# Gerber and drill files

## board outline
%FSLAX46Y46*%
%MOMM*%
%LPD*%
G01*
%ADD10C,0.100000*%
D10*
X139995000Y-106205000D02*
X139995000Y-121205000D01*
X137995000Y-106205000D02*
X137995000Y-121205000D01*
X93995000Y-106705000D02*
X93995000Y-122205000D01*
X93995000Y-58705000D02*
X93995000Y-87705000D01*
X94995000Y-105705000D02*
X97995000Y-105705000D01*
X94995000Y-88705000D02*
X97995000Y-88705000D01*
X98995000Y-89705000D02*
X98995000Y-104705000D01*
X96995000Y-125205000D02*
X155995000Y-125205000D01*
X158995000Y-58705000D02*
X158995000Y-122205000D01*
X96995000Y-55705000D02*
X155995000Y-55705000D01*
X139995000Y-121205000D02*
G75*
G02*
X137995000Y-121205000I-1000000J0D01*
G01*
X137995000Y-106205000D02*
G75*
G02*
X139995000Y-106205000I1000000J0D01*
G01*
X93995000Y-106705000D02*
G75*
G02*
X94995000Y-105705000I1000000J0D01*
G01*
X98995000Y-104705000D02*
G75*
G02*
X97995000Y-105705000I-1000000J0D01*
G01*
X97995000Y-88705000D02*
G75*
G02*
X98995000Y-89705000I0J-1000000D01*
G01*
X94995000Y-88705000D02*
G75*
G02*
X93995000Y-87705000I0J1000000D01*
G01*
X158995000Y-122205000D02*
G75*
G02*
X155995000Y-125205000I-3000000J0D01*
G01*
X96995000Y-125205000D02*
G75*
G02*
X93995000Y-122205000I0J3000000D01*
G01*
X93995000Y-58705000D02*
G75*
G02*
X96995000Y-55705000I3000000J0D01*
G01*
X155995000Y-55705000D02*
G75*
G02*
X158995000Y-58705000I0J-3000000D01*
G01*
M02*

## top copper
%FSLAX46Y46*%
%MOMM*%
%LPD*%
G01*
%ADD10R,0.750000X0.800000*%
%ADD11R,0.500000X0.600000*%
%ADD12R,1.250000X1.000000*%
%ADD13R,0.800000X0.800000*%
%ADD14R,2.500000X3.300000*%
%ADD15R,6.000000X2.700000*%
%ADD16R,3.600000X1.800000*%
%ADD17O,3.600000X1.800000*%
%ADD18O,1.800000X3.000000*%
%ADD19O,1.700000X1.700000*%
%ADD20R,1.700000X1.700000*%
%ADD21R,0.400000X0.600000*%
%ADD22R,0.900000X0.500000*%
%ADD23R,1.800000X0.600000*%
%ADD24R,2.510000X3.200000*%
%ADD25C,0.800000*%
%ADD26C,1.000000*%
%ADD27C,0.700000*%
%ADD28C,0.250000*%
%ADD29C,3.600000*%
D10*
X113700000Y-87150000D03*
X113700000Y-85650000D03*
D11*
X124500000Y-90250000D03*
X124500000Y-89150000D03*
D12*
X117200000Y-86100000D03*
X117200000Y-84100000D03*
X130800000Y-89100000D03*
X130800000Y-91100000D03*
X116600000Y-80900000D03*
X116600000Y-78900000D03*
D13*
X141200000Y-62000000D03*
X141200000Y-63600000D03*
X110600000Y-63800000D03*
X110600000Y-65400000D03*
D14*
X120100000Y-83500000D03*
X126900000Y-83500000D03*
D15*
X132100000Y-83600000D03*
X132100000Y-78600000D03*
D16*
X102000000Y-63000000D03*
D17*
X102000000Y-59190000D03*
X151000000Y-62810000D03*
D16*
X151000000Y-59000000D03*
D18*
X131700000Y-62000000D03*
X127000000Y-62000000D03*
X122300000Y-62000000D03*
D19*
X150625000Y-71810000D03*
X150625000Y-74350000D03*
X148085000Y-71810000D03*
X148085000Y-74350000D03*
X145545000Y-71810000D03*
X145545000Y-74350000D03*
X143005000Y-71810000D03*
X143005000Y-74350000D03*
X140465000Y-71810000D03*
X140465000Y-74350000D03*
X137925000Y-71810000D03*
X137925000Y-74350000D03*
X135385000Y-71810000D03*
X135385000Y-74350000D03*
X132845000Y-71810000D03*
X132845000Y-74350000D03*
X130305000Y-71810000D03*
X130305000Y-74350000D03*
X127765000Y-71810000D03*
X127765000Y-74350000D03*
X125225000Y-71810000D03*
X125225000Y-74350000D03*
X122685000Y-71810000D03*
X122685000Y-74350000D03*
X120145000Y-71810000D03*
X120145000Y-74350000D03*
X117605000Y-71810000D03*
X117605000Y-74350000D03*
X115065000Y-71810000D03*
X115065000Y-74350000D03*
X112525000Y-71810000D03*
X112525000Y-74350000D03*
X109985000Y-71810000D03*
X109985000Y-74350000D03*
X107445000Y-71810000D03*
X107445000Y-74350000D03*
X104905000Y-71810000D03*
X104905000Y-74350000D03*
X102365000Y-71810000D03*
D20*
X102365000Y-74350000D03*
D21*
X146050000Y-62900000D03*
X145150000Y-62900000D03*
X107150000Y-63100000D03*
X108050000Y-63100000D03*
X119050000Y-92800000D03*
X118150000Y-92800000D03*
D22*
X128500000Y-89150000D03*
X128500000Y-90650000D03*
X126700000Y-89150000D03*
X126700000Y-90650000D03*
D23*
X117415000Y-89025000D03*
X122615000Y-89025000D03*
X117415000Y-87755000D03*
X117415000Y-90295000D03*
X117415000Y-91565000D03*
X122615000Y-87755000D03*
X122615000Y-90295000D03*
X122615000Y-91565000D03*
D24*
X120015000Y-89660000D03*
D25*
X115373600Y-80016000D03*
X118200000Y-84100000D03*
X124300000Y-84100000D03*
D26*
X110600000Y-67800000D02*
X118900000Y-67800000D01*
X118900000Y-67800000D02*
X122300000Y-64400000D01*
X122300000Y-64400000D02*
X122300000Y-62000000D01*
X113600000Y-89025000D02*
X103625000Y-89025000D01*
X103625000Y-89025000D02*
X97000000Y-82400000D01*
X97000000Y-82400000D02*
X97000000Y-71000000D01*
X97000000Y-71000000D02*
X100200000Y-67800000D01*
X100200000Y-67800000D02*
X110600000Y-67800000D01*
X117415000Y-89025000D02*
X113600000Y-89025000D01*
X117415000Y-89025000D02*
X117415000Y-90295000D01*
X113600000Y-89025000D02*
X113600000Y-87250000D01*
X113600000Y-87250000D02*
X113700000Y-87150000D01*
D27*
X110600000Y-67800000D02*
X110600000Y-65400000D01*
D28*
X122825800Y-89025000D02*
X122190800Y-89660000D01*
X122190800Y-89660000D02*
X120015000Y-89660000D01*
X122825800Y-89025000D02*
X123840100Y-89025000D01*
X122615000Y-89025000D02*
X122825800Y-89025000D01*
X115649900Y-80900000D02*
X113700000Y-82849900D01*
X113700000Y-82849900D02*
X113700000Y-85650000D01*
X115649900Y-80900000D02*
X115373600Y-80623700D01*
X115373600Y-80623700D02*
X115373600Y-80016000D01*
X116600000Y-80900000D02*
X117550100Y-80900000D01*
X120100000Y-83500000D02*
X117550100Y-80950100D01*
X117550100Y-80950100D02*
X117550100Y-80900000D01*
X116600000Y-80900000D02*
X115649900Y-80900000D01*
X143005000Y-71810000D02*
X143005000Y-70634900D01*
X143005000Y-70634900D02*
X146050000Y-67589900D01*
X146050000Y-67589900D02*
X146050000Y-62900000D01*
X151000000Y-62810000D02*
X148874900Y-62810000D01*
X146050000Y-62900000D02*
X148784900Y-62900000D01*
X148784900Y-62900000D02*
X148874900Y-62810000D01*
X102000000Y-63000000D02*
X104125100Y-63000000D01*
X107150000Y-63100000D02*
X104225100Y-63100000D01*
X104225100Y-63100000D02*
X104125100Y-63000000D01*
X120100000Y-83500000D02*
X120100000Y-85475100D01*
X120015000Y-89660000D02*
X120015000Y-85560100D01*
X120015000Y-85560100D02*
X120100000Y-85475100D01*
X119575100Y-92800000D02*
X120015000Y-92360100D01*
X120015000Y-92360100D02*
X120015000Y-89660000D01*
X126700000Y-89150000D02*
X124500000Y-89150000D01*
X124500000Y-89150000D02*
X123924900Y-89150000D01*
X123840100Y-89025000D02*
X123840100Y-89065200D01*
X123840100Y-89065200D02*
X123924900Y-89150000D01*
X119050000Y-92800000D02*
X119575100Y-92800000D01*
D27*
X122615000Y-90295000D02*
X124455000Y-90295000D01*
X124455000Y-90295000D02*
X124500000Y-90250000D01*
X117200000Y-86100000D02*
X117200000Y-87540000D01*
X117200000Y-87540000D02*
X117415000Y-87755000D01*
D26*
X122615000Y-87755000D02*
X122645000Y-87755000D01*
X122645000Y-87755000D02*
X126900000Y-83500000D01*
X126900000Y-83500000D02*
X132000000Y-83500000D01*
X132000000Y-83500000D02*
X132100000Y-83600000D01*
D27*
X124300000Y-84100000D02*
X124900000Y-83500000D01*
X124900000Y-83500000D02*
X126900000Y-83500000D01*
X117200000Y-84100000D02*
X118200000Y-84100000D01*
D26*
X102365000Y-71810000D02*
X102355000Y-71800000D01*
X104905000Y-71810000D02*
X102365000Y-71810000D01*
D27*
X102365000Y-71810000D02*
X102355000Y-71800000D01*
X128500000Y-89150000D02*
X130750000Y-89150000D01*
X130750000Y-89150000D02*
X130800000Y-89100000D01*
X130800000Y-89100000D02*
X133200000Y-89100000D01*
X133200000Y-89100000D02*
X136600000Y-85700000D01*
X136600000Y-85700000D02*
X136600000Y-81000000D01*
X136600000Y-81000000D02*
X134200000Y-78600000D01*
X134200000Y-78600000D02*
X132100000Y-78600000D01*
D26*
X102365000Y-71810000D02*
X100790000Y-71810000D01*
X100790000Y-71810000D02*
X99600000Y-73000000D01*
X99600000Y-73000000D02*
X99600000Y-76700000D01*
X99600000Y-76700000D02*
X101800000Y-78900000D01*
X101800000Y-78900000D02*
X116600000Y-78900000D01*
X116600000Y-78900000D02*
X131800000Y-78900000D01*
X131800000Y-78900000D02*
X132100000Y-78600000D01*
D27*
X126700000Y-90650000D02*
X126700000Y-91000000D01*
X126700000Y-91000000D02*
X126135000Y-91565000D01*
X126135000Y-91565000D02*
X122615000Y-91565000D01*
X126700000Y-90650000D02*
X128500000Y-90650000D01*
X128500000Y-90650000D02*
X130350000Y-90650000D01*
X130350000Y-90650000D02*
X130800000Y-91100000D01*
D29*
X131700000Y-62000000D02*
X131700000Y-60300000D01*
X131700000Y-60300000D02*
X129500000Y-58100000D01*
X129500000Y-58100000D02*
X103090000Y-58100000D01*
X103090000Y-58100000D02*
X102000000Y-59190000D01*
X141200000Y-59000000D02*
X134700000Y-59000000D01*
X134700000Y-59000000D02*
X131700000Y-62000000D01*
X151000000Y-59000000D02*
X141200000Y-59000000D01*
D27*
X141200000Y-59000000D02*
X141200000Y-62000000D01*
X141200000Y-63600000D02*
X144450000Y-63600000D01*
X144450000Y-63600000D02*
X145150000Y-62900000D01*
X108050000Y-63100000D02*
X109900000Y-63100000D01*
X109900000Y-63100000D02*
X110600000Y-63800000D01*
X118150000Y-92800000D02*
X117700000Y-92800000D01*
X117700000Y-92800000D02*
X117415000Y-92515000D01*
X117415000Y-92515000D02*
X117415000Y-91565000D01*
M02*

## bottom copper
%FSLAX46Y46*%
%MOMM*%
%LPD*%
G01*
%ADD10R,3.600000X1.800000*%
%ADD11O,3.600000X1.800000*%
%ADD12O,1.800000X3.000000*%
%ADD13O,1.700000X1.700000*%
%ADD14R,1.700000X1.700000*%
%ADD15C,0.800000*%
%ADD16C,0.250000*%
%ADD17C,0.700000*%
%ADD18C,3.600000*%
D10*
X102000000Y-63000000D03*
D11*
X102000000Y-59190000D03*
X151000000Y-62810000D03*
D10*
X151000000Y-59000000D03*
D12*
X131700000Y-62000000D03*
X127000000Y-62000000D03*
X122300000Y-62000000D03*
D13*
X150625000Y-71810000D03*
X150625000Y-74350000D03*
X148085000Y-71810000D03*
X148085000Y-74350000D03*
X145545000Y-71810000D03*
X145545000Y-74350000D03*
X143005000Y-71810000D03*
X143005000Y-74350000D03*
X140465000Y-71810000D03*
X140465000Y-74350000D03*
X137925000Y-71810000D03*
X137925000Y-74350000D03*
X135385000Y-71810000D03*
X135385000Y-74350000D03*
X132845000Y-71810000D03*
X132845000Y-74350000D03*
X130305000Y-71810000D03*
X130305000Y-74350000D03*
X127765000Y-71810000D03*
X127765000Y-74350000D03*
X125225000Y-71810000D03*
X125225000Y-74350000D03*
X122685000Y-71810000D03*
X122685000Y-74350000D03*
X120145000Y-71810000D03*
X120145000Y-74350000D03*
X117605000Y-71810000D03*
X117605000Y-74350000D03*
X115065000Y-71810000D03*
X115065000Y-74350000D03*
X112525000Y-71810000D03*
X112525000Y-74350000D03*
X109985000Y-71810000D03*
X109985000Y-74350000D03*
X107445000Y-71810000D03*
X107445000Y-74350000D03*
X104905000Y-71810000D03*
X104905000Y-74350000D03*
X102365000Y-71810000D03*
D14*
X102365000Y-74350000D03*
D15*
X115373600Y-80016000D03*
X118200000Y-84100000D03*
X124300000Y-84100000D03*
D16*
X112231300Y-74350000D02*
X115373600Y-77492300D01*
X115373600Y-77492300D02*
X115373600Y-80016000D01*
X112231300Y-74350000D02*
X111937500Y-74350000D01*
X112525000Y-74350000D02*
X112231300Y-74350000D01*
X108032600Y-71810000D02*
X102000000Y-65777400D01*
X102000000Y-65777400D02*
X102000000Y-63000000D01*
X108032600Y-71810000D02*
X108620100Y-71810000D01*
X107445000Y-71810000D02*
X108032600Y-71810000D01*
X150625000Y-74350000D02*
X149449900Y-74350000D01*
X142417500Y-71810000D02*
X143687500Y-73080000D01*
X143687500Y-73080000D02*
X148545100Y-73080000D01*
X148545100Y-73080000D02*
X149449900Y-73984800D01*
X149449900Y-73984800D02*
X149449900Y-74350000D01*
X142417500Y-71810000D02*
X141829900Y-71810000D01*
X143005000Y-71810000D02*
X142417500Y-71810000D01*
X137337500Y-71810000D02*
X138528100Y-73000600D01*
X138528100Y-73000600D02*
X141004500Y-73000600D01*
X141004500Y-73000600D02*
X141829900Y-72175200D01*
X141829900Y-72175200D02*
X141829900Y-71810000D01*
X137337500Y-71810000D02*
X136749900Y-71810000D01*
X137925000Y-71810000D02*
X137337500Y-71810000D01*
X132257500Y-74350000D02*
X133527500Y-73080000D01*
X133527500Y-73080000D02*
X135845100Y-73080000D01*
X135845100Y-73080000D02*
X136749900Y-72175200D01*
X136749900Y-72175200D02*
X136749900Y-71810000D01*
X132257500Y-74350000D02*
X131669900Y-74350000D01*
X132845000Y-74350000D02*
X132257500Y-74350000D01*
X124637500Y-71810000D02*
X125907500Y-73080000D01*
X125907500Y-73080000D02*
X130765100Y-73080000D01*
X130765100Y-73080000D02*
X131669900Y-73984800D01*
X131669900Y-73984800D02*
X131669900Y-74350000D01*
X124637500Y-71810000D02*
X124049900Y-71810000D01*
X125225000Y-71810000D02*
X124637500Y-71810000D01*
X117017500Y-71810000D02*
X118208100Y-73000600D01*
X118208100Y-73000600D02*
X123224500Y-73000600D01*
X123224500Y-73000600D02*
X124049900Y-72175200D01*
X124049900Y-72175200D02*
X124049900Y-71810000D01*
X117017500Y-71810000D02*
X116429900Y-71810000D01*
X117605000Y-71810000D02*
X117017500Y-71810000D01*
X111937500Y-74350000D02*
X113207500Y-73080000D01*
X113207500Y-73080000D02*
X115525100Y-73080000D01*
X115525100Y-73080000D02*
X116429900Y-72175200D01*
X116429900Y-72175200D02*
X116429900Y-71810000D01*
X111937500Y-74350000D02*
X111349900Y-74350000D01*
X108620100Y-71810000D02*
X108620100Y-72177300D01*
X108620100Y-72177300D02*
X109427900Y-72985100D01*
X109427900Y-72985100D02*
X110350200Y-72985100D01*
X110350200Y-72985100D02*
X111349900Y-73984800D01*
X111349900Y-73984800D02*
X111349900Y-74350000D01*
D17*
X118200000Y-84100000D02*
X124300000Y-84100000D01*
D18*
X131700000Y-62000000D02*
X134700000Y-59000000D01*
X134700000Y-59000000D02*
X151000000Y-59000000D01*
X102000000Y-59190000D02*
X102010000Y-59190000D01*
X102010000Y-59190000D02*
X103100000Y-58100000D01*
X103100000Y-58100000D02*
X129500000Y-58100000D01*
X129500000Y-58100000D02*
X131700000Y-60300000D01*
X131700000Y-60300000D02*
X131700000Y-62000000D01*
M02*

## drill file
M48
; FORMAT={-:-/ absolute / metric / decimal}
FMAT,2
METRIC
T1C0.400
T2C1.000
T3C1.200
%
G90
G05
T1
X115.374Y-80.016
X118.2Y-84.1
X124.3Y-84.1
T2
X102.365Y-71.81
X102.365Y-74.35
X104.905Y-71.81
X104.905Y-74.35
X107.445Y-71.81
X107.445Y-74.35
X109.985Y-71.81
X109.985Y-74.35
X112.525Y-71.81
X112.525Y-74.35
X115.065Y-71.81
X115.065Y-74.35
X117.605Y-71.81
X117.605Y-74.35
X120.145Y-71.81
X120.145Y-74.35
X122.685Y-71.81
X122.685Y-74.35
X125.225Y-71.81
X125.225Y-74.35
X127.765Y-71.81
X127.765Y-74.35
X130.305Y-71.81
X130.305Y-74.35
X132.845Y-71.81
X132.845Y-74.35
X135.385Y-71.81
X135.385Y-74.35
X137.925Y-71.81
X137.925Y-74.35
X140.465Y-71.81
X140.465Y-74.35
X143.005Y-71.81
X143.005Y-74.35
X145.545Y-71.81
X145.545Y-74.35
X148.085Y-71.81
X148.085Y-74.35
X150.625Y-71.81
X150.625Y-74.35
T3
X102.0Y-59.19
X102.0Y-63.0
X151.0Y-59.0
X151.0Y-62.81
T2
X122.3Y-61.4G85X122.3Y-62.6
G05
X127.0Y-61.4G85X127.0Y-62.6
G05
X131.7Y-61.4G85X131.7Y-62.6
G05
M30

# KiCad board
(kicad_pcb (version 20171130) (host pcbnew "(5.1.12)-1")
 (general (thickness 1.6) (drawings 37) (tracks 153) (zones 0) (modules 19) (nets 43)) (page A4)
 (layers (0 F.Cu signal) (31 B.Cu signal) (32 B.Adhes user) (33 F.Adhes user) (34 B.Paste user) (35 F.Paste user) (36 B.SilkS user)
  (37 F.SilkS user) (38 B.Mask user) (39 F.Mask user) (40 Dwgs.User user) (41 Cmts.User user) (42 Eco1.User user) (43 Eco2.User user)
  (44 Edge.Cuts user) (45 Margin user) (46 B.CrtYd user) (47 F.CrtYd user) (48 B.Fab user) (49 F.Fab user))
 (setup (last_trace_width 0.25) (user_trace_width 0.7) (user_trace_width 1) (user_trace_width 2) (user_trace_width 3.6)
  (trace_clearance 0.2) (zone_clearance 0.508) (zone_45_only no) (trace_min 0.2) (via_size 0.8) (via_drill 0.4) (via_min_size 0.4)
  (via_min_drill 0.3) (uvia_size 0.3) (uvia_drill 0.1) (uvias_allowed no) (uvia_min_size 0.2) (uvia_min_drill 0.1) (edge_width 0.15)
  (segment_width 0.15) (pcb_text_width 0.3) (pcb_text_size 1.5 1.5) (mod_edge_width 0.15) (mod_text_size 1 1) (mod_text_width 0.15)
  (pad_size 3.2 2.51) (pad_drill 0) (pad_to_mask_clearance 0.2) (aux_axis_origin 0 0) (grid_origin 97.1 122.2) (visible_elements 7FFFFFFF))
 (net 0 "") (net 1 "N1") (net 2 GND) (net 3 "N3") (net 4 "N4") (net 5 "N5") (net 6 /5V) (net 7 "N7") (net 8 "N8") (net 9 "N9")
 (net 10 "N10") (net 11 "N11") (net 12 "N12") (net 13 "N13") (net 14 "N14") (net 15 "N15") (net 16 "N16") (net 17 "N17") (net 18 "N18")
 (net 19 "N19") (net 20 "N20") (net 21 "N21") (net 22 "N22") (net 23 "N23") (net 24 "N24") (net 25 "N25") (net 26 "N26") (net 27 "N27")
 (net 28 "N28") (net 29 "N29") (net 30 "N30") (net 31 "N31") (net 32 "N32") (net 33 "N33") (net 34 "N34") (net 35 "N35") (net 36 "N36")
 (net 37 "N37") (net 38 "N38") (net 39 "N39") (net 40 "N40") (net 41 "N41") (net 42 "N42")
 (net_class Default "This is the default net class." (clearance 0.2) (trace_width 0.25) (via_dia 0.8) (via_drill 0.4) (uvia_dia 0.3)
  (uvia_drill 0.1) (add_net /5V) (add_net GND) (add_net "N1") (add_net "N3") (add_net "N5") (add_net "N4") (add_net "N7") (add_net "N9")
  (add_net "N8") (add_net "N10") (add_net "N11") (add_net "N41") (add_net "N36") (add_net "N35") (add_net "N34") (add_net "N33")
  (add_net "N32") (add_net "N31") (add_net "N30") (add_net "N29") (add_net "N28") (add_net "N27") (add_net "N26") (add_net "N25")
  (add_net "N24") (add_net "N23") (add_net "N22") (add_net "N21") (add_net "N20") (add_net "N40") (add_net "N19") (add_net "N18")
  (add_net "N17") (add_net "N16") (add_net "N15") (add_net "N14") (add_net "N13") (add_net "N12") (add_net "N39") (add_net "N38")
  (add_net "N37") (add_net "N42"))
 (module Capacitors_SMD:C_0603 (layer F.Cu) (at 113.7 86.4 270)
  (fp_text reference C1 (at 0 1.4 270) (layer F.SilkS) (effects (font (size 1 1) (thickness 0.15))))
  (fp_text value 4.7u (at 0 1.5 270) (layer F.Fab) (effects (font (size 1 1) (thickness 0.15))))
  (pad 2 smd rect (at 0.75 0 270) (size 0.8 0.75) (layers F.Cu F.Paste F.Mask) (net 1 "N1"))
  (pad 1 smd rect (at -0.75 0 270) (size 0.8 0.75) (layers F.Cu F.Paste F.Mask) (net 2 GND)))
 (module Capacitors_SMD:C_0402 (layer F.Cu) (at 124.5 89.7 270)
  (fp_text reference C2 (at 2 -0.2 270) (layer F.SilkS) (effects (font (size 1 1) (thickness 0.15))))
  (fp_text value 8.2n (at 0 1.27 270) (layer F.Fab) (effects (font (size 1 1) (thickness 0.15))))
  (pad 2 smd rect (at 0.55 0 270) (size 0.6 0.5) (layers F.Cu F.Paste F.Mask) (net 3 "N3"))
  (pad 1 smd rect (at -0.55 0 270) (size 0.6 0.5) (layers F.Cu F.Paste F.Mask) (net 2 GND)))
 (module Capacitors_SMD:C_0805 (layer F.Cu) (at 117.2 85.1 270)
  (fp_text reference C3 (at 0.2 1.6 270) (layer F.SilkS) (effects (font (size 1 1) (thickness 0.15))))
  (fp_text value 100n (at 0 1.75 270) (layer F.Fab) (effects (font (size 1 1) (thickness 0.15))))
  (pad 2 smd rect (at 1 0 270) (size 1 1.25) (layers F.Cu F.Paste F.Mask) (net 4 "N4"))
  (pad 1 smd rect (at -1 0 270) (size 1 1.25) (layers F.Cu F.Paste F.Mask) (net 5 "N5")))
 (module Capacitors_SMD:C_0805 (layer F.Cu) (at 130.8 90.1 90)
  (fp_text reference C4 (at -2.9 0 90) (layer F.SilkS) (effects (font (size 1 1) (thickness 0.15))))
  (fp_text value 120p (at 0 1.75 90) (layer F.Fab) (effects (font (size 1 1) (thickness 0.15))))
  (pad 2 smd rect (at 1 0 90) (size 1 1.25) (layers F.Cu F.Paste F.Mask) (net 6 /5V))
  (pad 1 smd rect (at -1 0 90) (size 1 1.25) (layers F.Cu F.Paste F.Mask) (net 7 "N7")))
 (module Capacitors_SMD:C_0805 (layer F.Cu) (at 116.6 79.9 90)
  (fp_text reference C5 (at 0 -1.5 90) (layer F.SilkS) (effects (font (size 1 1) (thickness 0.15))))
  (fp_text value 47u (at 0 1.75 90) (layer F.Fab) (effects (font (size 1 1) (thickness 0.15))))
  (pad 1 smd rect (at -1 0 90) (size 1 1.25) (layers F.Cu F.Paste F.Mask) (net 2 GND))
  (pad 2 smd rect (at 1 0 90) (size 1 1.25) (layers F.Cu F.Paste F.Mask) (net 6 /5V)))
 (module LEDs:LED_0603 (layer F.Cu) (at 141.2 62.8 90)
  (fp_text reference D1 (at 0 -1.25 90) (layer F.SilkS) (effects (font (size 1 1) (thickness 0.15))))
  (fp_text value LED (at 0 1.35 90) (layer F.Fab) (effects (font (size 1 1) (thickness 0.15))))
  (pad 2 smd rect (at 0.8 0 270) (size 0.8 0.8) (layers F.Cu F.Paste F.Mask) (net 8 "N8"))
  (pad 1 smd rect (at -0.8 0 270) (size 0.8 0.8) (layers F.Cu F.Paste F.Mask) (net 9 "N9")))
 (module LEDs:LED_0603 (layer F.Cu) (at 110.6 64.6 270)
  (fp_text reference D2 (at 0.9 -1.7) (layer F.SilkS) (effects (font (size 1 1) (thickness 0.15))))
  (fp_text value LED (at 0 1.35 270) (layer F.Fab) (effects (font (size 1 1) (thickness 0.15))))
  (pad 1 smd rect (at -0.8 0 90) (size 0.8 0.8) (layers F.Cu F.Paste F.Mask) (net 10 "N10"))
  (pad 2 smd rect (at 0.8 0 90) (size 0.8 0.8) (layers F.Cu F.Paste F.Mask) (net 1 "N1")))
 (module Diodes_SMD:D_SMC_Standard (layer F.Cu) (at 123.5 83.5 180)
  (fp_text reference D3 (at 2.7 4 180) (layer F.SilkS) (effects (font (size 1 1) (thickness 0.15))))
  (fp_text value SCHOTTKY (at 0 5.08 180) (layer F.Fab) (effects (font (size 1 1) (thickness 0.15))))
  (pad 2 smd rect (at 3.4 0 270) (size 3.3 2.5) (layers F.Cu F.Paste F.Mask) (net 2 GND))
  (pad 1 smd rect (at -3.4 0 270) (size 3.3 2.5) (layers F.Cu F.Paste F.Mask) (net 5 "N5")))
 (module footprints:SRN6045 (layer F.Cu) (at 132.1 81.1 270)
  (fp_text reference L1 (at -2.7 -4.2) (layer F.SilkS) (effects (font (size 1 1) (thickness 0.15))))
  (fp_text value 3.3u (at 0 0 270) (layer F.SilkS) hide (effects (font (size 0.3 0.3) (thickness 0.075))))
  (pad 2 smd rect (at 2.5 0 270) (size 2.7 6) (layers F.Cu F.Paste F.Mask) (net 5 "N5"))
  (pad 1 smd rect (at -2.5 0 270) (size 2.7 6) (layers F.Cu F.Paste F.Mask) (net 6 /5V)))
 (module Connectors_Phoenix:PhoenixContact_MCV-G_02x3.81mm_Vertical (layer F.Cu) (at 102 63 90)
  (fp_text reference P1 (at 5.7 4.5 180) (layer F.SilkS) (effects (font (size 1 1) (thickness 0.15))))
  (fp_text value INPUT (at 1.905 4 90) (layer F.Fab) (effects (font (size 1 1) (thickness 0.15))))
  (pad 1 thru_hole rect (at 0 0 90) (size 1.8 3.6) (drill 1.2) (layers *.Cu *.Mask) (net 2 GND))
  (pad 2 thru_hole oval (at 3.81 0 90) (size 1.8 3.6) (drill 1.2) (layers *.Cu *.Mask) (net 8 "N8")))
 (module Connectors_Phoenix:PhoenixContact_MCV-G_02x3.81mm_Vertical (layer F.Cu) (at 151 59 270)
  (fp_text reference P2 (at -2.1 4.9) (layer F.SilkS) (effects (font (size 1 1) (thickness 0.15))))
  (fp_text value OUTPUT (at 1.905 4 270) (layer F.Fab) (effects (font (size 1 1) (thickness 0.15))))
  (pad 2 thru_hole oval (at 3.81 0 270) (size 1.8 3.6) (drill 1.2) (layers *.Cu *.Mask) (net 2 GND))
  (pad 1 thru_hole rect (at 0 0 270) (size 1.8 3.6) (drill 1.2) (layers *.Cu *.Mask) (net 8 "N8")))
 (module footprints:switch (layer F.Cu) (at 127 62)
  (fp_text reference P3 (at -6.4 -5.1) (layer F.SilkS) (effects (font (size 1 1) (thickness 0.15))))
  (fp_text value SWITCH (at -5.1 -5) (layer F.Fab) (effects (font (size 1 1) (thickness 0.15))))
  (pad 3 thru_hole oval (at 4.7 0) (size 1.8 3) (drill oval 1 2.2) (layers *.Cu *.Mask) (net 8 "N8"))
  (pad 2 thru_hole oval (at 0 0) (size 1.8 3) (drill oval 1 2.2) (layers *.Cu *.Mask) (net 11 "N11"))
  (pad 1 thru_hole oval (at -4.7 0) (size 1.8 3) (drill oval 1 2.2) (layers *.Cu *.Mask) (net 1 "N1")))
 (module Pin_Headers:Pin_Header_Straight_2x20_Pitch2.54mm (layer F.Cu) (at 102.365 74.35 90)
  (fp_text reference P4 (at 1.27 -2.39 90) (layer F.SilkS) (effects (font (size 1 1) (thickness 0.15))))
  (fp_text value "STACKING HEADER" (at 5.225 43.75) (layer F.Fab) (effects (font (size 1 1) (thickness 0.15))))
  (pad 40 thru_hole oval (at 2.54 48.26 90) (size 1.7 1.7) (drill 1) (layers *.Cu *.Mask) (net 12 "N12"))
  (pad 39 thru_hole oval (at 0 48.26 90) (size 1.7 1.7) (drill 1) (layers *.Cu *.Mask) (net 2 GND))
  (pad 38 thru_hole oval (at 2.54 45.72 90) (size 1.7 1.7) (drill 1) (layers *.Cu *.Mask) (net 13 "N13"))
  (pad 37 thru_hole oval (at 0 45.72 90) (size 1.7 1.7) (drill 1) (layers *.Cu *.Mask) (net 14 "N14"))
  (pad 36 thru_hole oval (at 2.54 43.18 90) (size 1.7 1.7) (drill 1) (layers *.Cu *.Mask) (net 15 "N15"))
  (pad 35 thru_hole oval (at 0 43.18 90) (size 1.7 1.7) (drill 1) (layers *.Cu *.Mask) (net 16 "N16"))
  (pad 34 thru_hole oval (at 2.54 40.64 90) (size 1.7 1.7) (drill 1) (layers *.Cu *.Mask) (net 2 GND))
  (pad 33 thru_hole oval (at 0 40.64 90) (size 1.7 1.7) (drill 1) (layers *.Cu *.Mask) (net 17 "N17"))
  (pad 32 thru_hole oval (at 2.54 38.1 90) (size 1.7 1.7) (drill 1) (layers *.Cu *.Mask) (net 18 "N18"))
  (pad 31 thru_hole oval (at 0 38.1 90) (size 1.7 1.7) (drill 1) (layers *.Cu *.Mask) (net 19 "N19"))
  (pad 30 thru_hole oval (at 2.54 35.56 90) (size 1.7 1.7) (drill 1) (layers *.Cu *.Mask) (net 2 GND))
  (pad 29 thru_hole oval (at 0 35.56 90) (size 1.7 1.7) (drill 1) (layers *.Cu *.Mask) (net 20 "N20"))
  (pad 28 thru_hole oval (at 2.54 33.02 90) (size 1.7 1.7) (drill 1) (layers *.Cu *.Mask) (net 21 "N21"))
  (pad 27 thru_hole oval (at 0 33.02 90) (size 1.7 1.7) (drill 1) (layers *.Cu *.Mask) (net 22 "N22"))
  (pad 26 thru_hole oval (at 2.54 30.48 90) (size 1.7 1.7) (drill 1) (layers *.Cu *.Mask) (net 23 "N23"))
  (pad 25 thru_hole oval (at 0 30.48 90) (size 1.7 1.7) (drill 1) (layers *.Cu *.Mask) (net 2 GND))
  (pad 24 thru_hole oval (at 2.54 27.94 90) (size 1.7 1.7) (drill 1) (layers *.Cu *.Mask) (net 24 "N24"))
  (pad 23 thru_hole oval (at 0 27.94 90) (size 1.7 1.7) (drill 1) (layers *.Cu *.Mask) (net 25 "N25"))
  (pad 22 thru_hole oval (at 2.54 25.4 90) (size 1.7 1.7) (drill 1) (layers *.Cu *.Mask) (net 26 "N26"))
  (pad 21 thru_hole oval (at 0 25.4 90) (size 1.7 1.7) (drill 1) (layers *.Cu *.Mask) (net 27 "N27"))
  (pad 20 thru_hole oval (at 2.54 22.86 90) (size 1.7 1.7) (drill 1) (layers *.Cu *.Mask) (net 2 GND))
  (pad 19 thru_hole oval (at 0 22.86 90) (size 1.7 1.7) (drill 1) (layers *.Cu *.Mask) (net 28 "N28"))
  (pad 18 thru_hole oval (at 2.54 20.32 90) (size 1.7 1.7) (drill 1) (layers *.Cu *.Mask) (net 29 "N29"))
  (pad 17 thru_hole oval (at 0 20.32 90) (size 1.7 1.7) (drill 1) (layers *.Cu *.Mask) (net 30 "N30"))
  (pad 16 thru_hole oval (at 2.54 17.78 90) (size 1.7 1.7) (drill 1) (layers *.Cu *.Mask) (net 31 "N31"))
  (pad 15 thru_hole oval (at 0 17.78 90) (size 1.7 1.7) (drill 1) (layers *.Cu *.Mask) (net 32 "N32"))
  (pad 14 thru_hole oval (at 2.54 15.24 90) (size 1.7 1.7) (drill 1) (layers *.Cu *.Mask) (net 2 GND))
  (pad 13 thru_hole oval (at 0 15.24 90) (size 1.7 1.7) (drill 1) (layers *.Cu *.Mask) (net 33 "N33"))
  (pad 12 thru_hole oval (at 2.54 12.7 90) (size 1.7 1.7) (drill 1) (layers *.Cu *.Mask) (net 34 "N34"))
  (pad 11 thru_hole oval (at 0 12.7 90) (size 1.7 1.7) (drill 1) (layers *.Cu *.Mask) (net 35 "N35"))
  (pad 10 thru_hole oval (at 2.54 10.16 90) (size 1.7 1.7) (drill 1) (layers *.Cu *.Mask) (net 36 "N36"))
  (pad 9 thru_hole oval (at 0 10.16 90) (size 1.7 1.7) (drill 1) (layers *.Cu *.Mask) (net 2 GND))
  (pad 8 thru_hole oval (at 2.54 7.62 90) (size 1.7 1.7) (drill 1) (layers *.Cu *.Mask) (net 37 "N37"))
  (pad 7 thru_hole oval (at 0 7.62 90) (size 1.7 1.7) (drill 1) (layers *.Cu *.Mask) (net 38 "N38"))
  (pad 6 thru_hole oval (at 2.54 5.08 90) (size 1.7 1.7) (drill 1) (layers *.Cu *.Mask) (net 2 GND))
  (pad 5 thru_hole oval (at 0 5.08 90) (size 1.7 1.7) (drill 1) (layers *.Cu *.Mask) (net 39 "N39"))
  (pad 4 thru_hole oval (at 2.54 2.54 90) (size 1.7 1.7) (drill 1) (layers *.Cu *.Mask) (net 6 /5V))
  (pad 3 thru_hole oval (at 0 2.54 90) (size 1.7 1.7) (drill 1) (layers *.Cu *.Mask) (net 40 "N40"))
  (pad 2 thru_hole oval (at 2.54 0 90) (size 1.7 1.7) (drill 1) (layers *.Cu *.Mask) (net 6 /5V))
  (pad 1 thru_hole rect (at 0 0 90) (size 1.7 1.7) (drill 1) (layers *.Cu *.Mask) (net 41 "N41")))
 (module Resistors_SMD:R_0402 (layer F.Cu) (at 145.6 62.9)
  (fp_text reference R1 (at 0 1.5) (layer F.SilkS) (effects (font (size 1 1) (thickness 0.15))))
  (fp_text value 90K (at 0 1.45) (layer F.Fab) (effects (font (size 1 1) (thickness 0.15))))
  (pad 2 smd rect (at 0.45 0) (size 0.4 0.6) (layers F.Cu F.Paste F.Mask) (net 2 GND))
  (pad 1 smd rect (at -0.45 0) (size 0.4 0.6) (layers F.Cu F.Paste F.Mask) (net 9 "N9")))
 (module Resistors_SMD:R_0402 (layer F.Cu) (at 107.6 63.1 180)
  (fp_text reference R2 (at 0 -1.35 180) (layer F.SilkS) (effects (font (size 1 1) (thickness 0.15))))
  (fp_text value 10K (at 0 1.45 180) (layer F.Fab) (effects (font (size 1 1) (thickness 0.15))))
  (pad 2 smd rect (at 0.45 0 180) (size 0.4 0.6) (layers F.Cu F.Paste F.Mask) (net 2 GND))
  (pad 1 smd rect (at -0.45 0 180) (size 0.4 0.6) (layers F.Cu F.Paste F.Mask) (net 10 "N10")))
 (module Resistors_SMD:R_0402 (layer F.Cu) (at 118.6 92.8)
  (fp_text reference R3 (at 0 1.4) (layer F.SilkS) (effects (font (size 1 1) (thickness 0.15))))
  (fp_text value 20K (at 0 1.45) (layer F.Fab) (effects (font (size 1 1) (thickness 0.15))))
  (pad 2 smd rect (at 0.45 0) (size 0.4 0.6) (layers F.Cu F.Paste F.Mask) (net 2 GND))
  (pad 1 smd rect (at -0.45 0) (size 0.4 0.6) (layers F.Cu F.Paste F.Mask) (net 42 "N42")))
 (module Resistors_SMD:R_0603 (layer F.Cu) (at 128.5 89.9 270)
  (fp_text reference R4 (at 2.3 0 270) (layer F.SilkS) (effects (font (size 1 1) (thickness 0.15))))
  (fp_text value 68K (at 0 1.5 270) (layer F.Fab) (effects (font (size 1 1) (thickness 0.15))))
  (pad 1 smd rect (at -0.75 0 270) (size 0.5 0.9) (layers F.Cu F.Paste F.Mask) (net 6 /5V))
  (pad 2 smd rect (at 0.75 0 270) (size 0.5 0.9) (layers F.Cu F.Paste F.Mask) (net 7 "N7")))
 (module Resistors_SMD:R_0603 (layer F.Cu) (at 126.7 89.9 90)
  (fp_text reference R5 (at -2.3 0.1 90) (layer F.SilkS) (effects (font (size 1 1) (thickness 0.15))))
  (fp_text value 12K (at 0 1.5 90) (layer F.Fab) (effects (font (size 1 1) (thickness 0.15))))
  (pad 2 smd rect (at 0.75 0 90) (size 0.5 0.9) (layers F.Cu F.Paste F.Mask) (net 2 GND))
  (pad 1 smd rect (at -0.75 0 90) (size 0.5 0.9) (layers F.Cu F.Paste F.Mask) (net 7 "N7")))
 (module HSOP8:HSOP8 (layer F.Cu) (at 120.015 89.66 270) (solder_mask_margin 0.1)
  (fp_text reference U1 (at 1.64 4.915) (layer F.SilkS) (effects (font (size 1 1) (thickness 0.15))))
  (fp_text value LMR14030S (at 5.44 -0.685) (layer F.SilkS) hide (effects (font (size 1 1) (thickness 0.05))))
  (pad 2 smd rect (at -0.635 2.6 270) (size 0.6 1.8) (layers F.Cu F.Paste F.Mask) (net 1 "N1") (solder_mask_margin 0.2))
  (pad 7 smd rect (at -0.635 -2.6 270) (size 0.6 1.8) (layers F.Cu F.Paste F.Mask) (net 2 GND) (solder_mask_margin 0.2))
  (pad 1 smd rect (at -1.905 2.6 270) (size 0.6 1.8) (layers F.Cu F.Paste F.Mask) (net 4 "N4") (solder_mask_margin 0.2))
  (pad 3 smd rect (at 0.635 2.6 270) (size 0.6 1.8) (layers F.Cu F.Paste F.Mask) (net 1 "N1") (solder_mask_margin 0.2))
  (pad 4 smd rect (at 1.905 2.6 270) (size 0.6 1.8) (layers F.Cu F.Paste F.Mask) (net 42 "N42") (solder_mask_margin 0.2))
  (pad 8 smd rect (at -1.905 -2.6 270) (size 0.6 1.8) (layers F.Cu F.Paste F.Mask) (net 5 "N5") (solder_mask_margin 0.2))
  (pad 6 smd rect (at 0.635 -2.6 270) (size 0.6 1.8) (layers F.Cu F.Paste F.Mask) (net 3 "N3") (solder_mask_margin 0.2))
  (pad 5 smd rect (at 1.905 -2.6 270) (size 0.6 1.8) (layers F.Cu F.Paste F.Mask) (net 7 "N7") (solder_mask_margin 0.2))
  (pad 9 smd rect (at 0 0 270) (size 3.2 2.51) (layers F.Cu F.Paste F.Mask) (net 2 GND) (solder_mask_margin 0.2)))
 (gr_line (start 139.995 106.205) (end 139.995 121.205) (angle 90) (layer Edge.Cuts) (width 0.1))
 (gr_line (start 137.995 106.205) (end 137.995 121.205) (angle 90) (layer Edge.Cuts) (width 0.1))
 (gr_line (start 93.995 106.705) (end 93.995 122.205) (layer Edge.Cuts) (width 0.1))
 (gr_line (start 93.995 58.705) (end 93.995 87.705) (layer Edge.Cuts) (width 0.1))
 (gr_line (start 94.995 105.705) (end 97.995 105.705) (layer Edge.Cuts) (width 0.1))
 (gr_line (start 94.995 88.705) (end 97.995 88.705) (layer Edge.Cuts) (width 0.1))
 (gr_line (start 98.995 89.705) (end 98.995 104.705) (layer Edge.Cuts) (width 0.1))
 (gr_line (start 96.995 125.205) (end 155.995 125.205) (angle 90) (layer Edge.Cuts) (width 0.1))
 (gr_line (start 158.995 58.705) (end 158.995 122.205) (angle 90) (layer Edge.Cuts) (width 0.1))
 (gr_line (start 96.995 55.705) (end 155.995 55.705) (angle 90) (layer Edge.Cuts) (width 0.1))
 (gr_arc (start 138.995 121.205) (end 137.995 121.205) (angle -180) (layer Edge.Cuts) (width 0.1))
 (gr_arc (start 138.995 106.205) (end 137.995 106.205) (angle 180) (layer Edge.Cuts) (width 0.1))
 (gr_arc (start 94.995 106.705) (end 93.995 106.705) (angle 90) (layer Edge.Cuts) (width 0.1))
 (gr_arc (start 97.995 104.705) (end 98.995 104.705) (angle 90) (layer Edge.Cuts) (width 0.1))
 (gr_arc (start 97.995 89.705) (end 97.995 88.705) (angle 90) (layer Edge.Cuts) (width 0.1))
 (gr_arc (start 94.995 87.705) (end 94.995 88.705) (angle 90) (layer Edge.Cuts) (width 0.1))
 (gr_arc (start 155.995 122.205) (end 158.995 122.205) (angle 90) (layer Edge.Cuts) (width 0.1))
 (gr_arc (start 96.995 122.205) (end 96.995 125.205) (angle 90) (layer Edge.Cuts) (width 0.1))
 (gr_arc (start 96.995 58.705) (end 93.995 58.705) (angle 90) (layer Edge.Cuts) (width 0.1))
 (gr_arc (start 155.995 58.705) (end 155.995 55.705) (angle 90) (layer Edge.Cuts) (width 0.1))
 (segment (start 110.6 67.8) (end 118.9 67.8) (width 1) (layer F.Cu) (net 1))
 (segment (start 118.9 67.8) (end 122.3 64.4) (width 1) (layer F.Cu) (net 1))
 (segment (start 122.3 64.4) (end 122.3 62) (width 1) (layer F.Cu) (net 1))
 (segment (start 113.6 89.025) (end 103.625 89.025) (width 1) (layer F.Cu) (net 1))
 (segment (start 103.625 89.025) (end 97 82.4) (width 1) (layer F.Cu) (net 1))
 (segment (start 97 82.4) (end 97 71) (width 1) (layer F.Cu) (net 1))
 (segment (start 97 71) (end 100.2 67.8) (width 1) (layer F.Cu) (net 1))
 (segment (start 100.2 67.8) (end 110.6 67.8) (width 1) (layer F.Cu) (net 1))
 (segment (start 117.415 89.025) (end 113.6 89.025) (width 1) (layer F.Cu) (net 1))
 (segment (start 117.415 89.025) (end 117.415 90.295) (width 1) (layer F.Cu) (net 1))
 (segment (start 113.6 89.025) (end 113.6 87.25) (width 1) (layer F.Cu) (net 1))
 (segment (start 113.6 87.25) (end 113.7 87.15) (width 1) (layer F.Cu) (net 1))
 (segment (start 110.6 67.8) (end 110.6 65.4) (width 0.7) (layer F.Cu) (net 1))
 (segment (start 122.8258 89.025) (end 122.1908 89.66) (width 0.25) (layer F.Cu) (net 2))
 (segment (start 122.1908 89.66) (end 120.015 89.66) (width 0.25) (layer F.Cu) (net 2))
 (segment (start 122.8258 89.025) (end 123.8401 89.025) (width 0.25) (layer F.Cu) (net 2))
 (segment (start 122.615 89.025) (end 122.8258 89.025) (width 0.25) (layer F.Cu) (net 2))
 (segment (start 115.6499 80.9) (end 113.7 82.8499) (width 0.25) (layer F.Cu) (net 2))
 (segment (start 113.7 82.8499) (end 113.7 85.65) (width 0.25) (layer F.Cu) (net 2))
 (segment (start 115.6499 80.9) (end 115.3736 80.6237) (width 0.25) (layer F.Cu) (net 2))
 (segment (start 115.3736 80.6237) (end 115.3736 80.016) (width 0.25) (layer F.Cu) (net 2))
 (segment (start 116.6 80.9) (end 117.5501 80.9) (width 0.25) (layer F.Cu) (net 2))
 (segment (start 120.1 83.5) (end 117.5501 80.9501) (width 0.25) (layer F.Cu) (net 2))
 (segment (start 117.5501 80.9501) (end 117.5501 80.9) (width 0.25) (layer F.Cu) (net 2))
 (segment (start 112.2313 74.35) (end 115.3736 77.4923) (width 0.25) (layer B.Cu) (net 2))
 (segment (start 115.3736 77.4923) (end 115.3736 80.016) (width 0.25) (layer B.Cu) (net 2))
 (segment (start 116.6 80.9) (end 115.6499 80.9) (width 0.25) (layer F.Cu) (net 2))
 (segment (start 112.2313 74.35) (end 111.9375 74.35) (width 0.25) (layer B.Cu) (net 2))
 (segment (start 112.525 74.35) (end 112.2313 74.35) (width 0.25) (layer B.Cu) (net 2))
 (segment (start 108.0326 71.81) (end 102 65.7774) (width 0.25) (layer B.Cu) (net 2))
 (segment (start 102 65.7774) (end 102 63) (width 0.25) (layer B.Cu) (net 2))
 (segment (start 108.0326 71.81) (end 108.6201 71.81) (width 0.25) (layer B.Cu) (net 2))
 (segment (start 107.445 71.81) (end 108.0326 71.81) (width 0.25) (layer B.Cu) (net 2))
 (segment (start 143.005 71.81) (end 143.005 70.6349) (width 0.25) (layer F.Cu) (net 2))
 (segment (start 143.005 70.6349) (end 146.05 67.5899) (width 0.25) (layer F.Cu) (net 2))
 (segment (start 146.05 67.5899) (end 146.05 62.9) (width 0.25) (layer F.Cu) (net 2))
 (segment (start 150.625 74.35) (end 149.4499 74.35) (width 0.25) (layer B.Cu) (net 2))
 (segment (start 142.4175 71.81) (end 143.6875 73.08) (width 0.25) (layer B.Cu) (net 2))
 (segment (start 143.6875 73.08) (end 148.5451 73.08) (width 0.25) (layer B.Cu) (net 2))
 (segment (start 148.5451 73.08) (end 149.4499 73.9848) (width 0.25) (layer B.Cu) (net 2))
 (segment (start 149.4499 73.9848) (end 149.4499 74.35) (width 0.25) (layer B.Cu) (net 2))
 (segment (start 142.4175 71.81) (end 141.8299 71.81) (width 0.25) (layer B.Cu) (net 2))
 (segment (start 143.005 71.81) (end 142.4175 71.81) (width 0.25) (layer B.Cu) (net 2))
 (segment (start 137.3375 71.81) (end 138.5281 73.0006) (width 0.25) (layer B.Cu) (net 2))
 (segment (start 138.5281 73.0006) (end 141.0045 73.0006) (width 0.25) (layer B.Cu) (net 2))
 (segment (start 141.0045 73.0006) (end 141.8299 72.1752) (width 0.25) (layer B.Cu) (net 2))
 (segment (start 141.8299 72.1752) (end 141.8299 71.81) (width 0.25) (layer B.Cu) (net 2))
 (segment (start 137.3375 71.81) (end 136.7499 71.81) (width 0.25) (layer B.Cu) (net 2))
 (segment (start 137.925 71.81) (end 137.3375 71.81) (width 0.25) (layer B.Cu) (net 2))
 (segment (start 132.2575 74.35) (end 133.5275 73.08) (width 0.25) (layer B.Cu) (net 2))
 (segment (start 133.5275 73.08) (end 135.8451 73.08) (width 0.25) (layer B.Cu) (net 2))
 (segment (start 135.8451 73.08) (end 136.7499 72.1752) (width 0.25) (layer B.Cu) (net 2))
 (segment (start 136.7499 72.1752) (end 136.7499 71.81) (width 0.25) (layer B.Cu) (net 2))
 (segment (start 132.2575 74.35) (end 131.6699 74.35) (width 0.25) (layer B.Cu) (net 2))
 (segment (start 132.845 74.35) (end 132.2575 74.35) (width 0.25) (layer B.Cu) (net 2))
 (segment (start 124.6375 71.81) (end 125.9075 73.08) (width 0.25) (layer B.Cu) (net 2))
 (segment (start 125.9075 73.08) (end 130.7651 73.08) (width 0.25) (layer B.Cu) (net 2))
 (segment (start 130.7651 73.08) (end 131.6699 73.9848) (width 0.25) (layer B.Cu) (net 2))
 (segment (start 131.6699 73.9848) (end 131.6699 74.35) (width 0.25) (layer B.Cu) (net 2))
 (segment (start 124.6375 71.81) (end 124.0499 71.81) (width 0.25) (layer B.Cu) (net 2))
 (segment (start 125.225 71.81) (end 124.6375 71.81) (width 0.25) (layer B.Cu) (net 2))
 (segment (start 117.0175 71.81) (end 118.2081 73.0006) (width 0.25) (layer B.Cu) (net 2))
 (segment (start 118.2081 73.0006) (end 123.2245 73.0006) (width 0.25) (layer B.Cu) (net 2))
 (segment (start 123.2245 73.0006) (end 124.0499 72.1752) (width 0.25) (layer B.Cu) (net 2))
 (segment (start 124.0499 72.1752) (end 124.0499 71.81) (width 0.25) (layer B.Cu) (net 2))
 (segment (start 117.0175 71.81) (end 116.4299 71.81) (width 0.25) (layer B.Cu) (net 2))
 (segment (start 117.605 71.81) (end 117.0175 71.81) (width 0.25) (layer B.Cu) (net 2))
 (segment (start 111.9375 74.35) (end 113.2075 73.08) (width 0.25) (layer B.Cu) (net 2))
 (segment (start 113.2075 73.08) (end 115.5251 73.08) (width 0.25) (layer B.Cu) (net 2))
 (segment (start 115.5251 73.08) (end 116.4299 72.1752) (width 0.25) (layer B.Cu) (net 2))
 (segment (start 116.4299 72.1752) (end 116.4299 71.81) (width 0.25) (layer B.Cu) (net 2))
 (segment (start 111.9375 74.35) (end 111.3499 74.35) (width 0.25) (layer B.Cu) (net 2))
 (segment (start 108.6201 71.81) (end 108.6201 72.1773) (width 0.25) (layer B.Cu) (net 2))
 (segment (start 108.6201 72.1773) (end 109.4279 72.9851) (width 0.25) (layer B.Cu) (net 2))
 (segment (start 109.4279 72.9851) (end 110.3502 72.9851) (width 0.25) (layer B.Cu) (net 2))
 (segment (start 110.3502 72.9851) (end 111.3499 73.9848) (width 0.25) (layer B.Cu) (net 2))
 (segment (start 111.3499 73.9848) (end 111.3499 74.35) (width 0.25) (layer B.Cu) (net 2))
 (segment (start 151 62.81) (end 148.8749 62.81) (width 0.25) (layer F.Cu) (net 2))
 (segment (start 146.05 62.9) (end 148.7849 62.9) (width 0.25) (layer F.Cu) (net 2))
 (segment (start 148.7849 62.9) (end 148.8749 62.81) (width 0.25) (layer F.Cu) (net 2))
 (segment (start 102 63) (end 104.1251 63) (width 0.25) (layer F.Cu) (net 2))
 (segment (start 107.15 63.1) (end 104.2251 63.1) (width 0.25) (layer F.Cu) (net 2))
 (segment (start 104.2251 63.1) (end 104.1251 63) (width 0.25) (layer F.Cu) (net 2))
 (segment (start 120.1 83.5) (end 120.1 85.4751) (width 0.25) (layer F.Cu) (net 2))
 (segment (start 120.015 89.66) (end 120.015 85.5601) (width 0.25) (layer F.Cu) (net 2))
 (segment (start 120.015 85.5601) (end 120.1 85.4751) (width 0.25) (layer F.Cu) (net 2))
 (segment (start 119.5751 92.8) (end 120.015 92.3601) (width 0.25) (layer F.Cu) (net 2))
 (segment (start 120.015 92.3601) (end 120.015 89.66) (width 0.25) (layer F.Cu) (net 2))
 (segment (start 126.7 89.15) (end 124.5 89.15) (width 0.25) (layer F.Cu) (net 2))
 (segment (start 124.5 89.15) (end 123.9249 89.15) (width 0.25) (layer F.Cu) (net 2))
 (segment (start 123.8401 89.025) (end 123.8401 89.0652) (width 0.25) (layer F.Cu) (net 2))
 (segment (start 123.8401 89.0652) (end 123.9249 89.15) (width 0.25) (layer F.Cu) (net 2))
 (segment (start 119.05 92.8) (end 119.5751 92.8) (width 0.25) (layer F.Cu) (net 2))
 (via (at 115.3736 80.016) (size 0.8) (layers F.Cu B.Cu) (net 2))
 (segment (start 122.615 90.295) (end 124.455 90.295) (width 0.7) (layer F.Cu) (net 3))
 (segment (start 124.455 90.295) (end 124.5 90.25) (width 0.7) (layer F.Cu) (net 3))
 (segment (start 117.2 86.1) (end 117.2 87.54) (width 0.7) (layer F.Cu) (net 4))
 (segment (start 117.2 87.54) (end 117.415 87.755) (width 0.7) (layer F.Cu) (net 4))
 (segment (start 122.615 87.755) (end 122.645 87.755) (width 1) (layer F.Cu) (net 5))
 (segment (start 122.645 87.755) (end 126.9 83.5) (width 1) (layer F.Cu) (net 5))
 (segment (start 126.9 83.5) (end 132 83.5) (width 1) (layer F.Cu) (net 5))
 (segment (start 132 83.5) (end 132.1 83.6) (width 1) (layer F.Cu) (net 5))
 (segment (start 118.2 84.1) (end 124.3 84.1) (width 0.7) (layer B.Cu) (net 5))
 (segment (start 124.3 84.1) (end 124.9 83.5) (width 0.7) (layer F.Cu) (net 5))
 (segment (start 124.9 83.5) (end 126.9 83.5) (width 0.7) (layer F.Cu) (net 5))
 (segment (start 117.2 84.1) (end 118.2 84.1) (width 0.7) (layer F.Cu) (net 5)) (via (at 118.2 84.1) (size 0.8) (layers F.Cu B.Cu) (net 5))
 (via (at 124.3 84.1) (size 0.8) (layers F.Cu B.Cu) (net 5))
 (segment (start 102.365 71.81) (end 102.355 71.8) (width 1) (layer F.Cu) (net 6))
 (segment (start 104.905 71.81) (end 102.365 71.81) (width 1) (layer F.Cu) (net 6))
 (segment (start 102.365 71.81) (end 102.355 71.8) (width 0.7) (layer F.Cu) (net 6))
 (segment (start 128.5 89.15) (end 130.75 89.15) (width 0.7) (layer F.Cu) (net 6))
 (segment (start 130.75 89.15) (end 130.8 89.1) (width 0.7) (layer F.Cu) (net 6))
 (segment (start 130.8 89.1) (end 133.2 89.1) (width 0.7) (layer F.Cu) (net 6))
 (segment (start 133.2 89.1) (end 136.6 85.7) (width 0.7) (layer F.Cu) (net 6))
 (segment (start 136.6 85.7) (end 136.6 81) (width 0.7) (layer F.Cu) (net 6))
 (segment (start 136.6 81) (end 134.2 78.6) (width 0.7) (layer F.Cu) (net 6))
 (segment (start 134.2 78.6) (end 132.1 78.6) (width 0.7) (layer F.Cu) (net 6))
 (segment (start 102.365 71.81) (end 100.79 71.81) (width 1) (layer F.Cu) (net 6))
 (segment (start 100.79 71.81) (end 99.6 73) (width 1) (layer F.Cu) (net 6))
 (segment (start 99.6 73) (end 99.6 76.7) (width 1) (layer F.Cu) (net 6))
 (segment (start 99.6 76.7) (end 101.8 78.9) (width 1) (layer F.Cu) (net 6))
 (segment (start 101.8 78.9) (end 116.6 78.9) (width 1) (layer F.Cu) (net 6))
 (segment (start 116.6 78.9) (end 131.8 78.9) (width 1) (layer F.Cu) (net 6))
 (segment (start 131.8 78.9) (end 132.1 78.6) (width 1) (layer F.Cu) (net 6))
 (segment (start 126.7 90.65) (end 126.7 91) (width 0.7) (layer F.Cu) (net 7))
 (segment (start 126.7 91) (end 126.135 91.565) (width 0.7) (layer F.Cu) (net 7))
 (segment (start 126.135 91.565) (end 122.615 91.565) (width 0.7) (layer F.Cu) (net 7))
 (segment (start 126.7 90.65) (end 128.5 90.65) (width 0.7) (layer F.Cu) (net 7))
 (segment (start 128.5 90.65) (end 130.35 90.65) (width 0.7) (layer F.Cu) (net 7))
 (segment (start 130.35 90.65) (end 130.8 91.1) (width 0.7) (layer F.Cu) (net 7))
 (segment (start 131.7 62) (end 131.7 60.3) (width 3.6) (layer F.Cu) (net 8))
 (segment (start 131.7 60.3) (end 129.5 58.1) (width 3.6) (layer F.Cu) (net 8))
 (segment (start 129.5 58.1) (end 103.09 58.1) (width 3.6) (layer F.Cu) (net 8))
 (segment (start 103.09 58.1) (end 102 59.19) (width 3.6) (layer F.Cu) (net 8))
 (segment (start 141.2 59) (end 134.7 59) (width 3.6) (layer F.Cu) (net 8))
 (segment (start 134.7 59) (end 131.7 62) (width 3.6) (layer F.Cu) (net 8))
 (segment (start 151 59) (end 141.2 59) (width 3.6) (layer F.Cu) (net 8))
 (segment (start 141.2 59) (end 141.2 62) (width 0.7) (layer F.Cu) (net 8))
 (segment (start 131.7 62) (end 134.7 59) (width 3.6) (layer B.Cu) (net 8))
 (segment (start 134.7 59) (end 151 59) (width 3.6) (layer B.Cu) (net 8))
 (segment (start 102 59.19) (end 102.01 59.19) (width 3.6) (layer B.Cu) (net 8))
 (segment (start 102.01 59.19) (end 103.1 58.1) (width 3.6) (layer B.Cu) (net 8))
 (segment (start 103.1 58.1) (end 129.5 58.1) (width 3.6) (layer B.Cu) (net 8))
 (segment (start 129.5 58.1) (end 131.7 60.3) (width 3.6) (layer B.Cu) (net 8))
 (segment (start 131.7 60.3) (end 131.7 62) (width 3.6) (layer B.Cu) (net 8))
 (segment (start 141.2 63.6) (end 144.45 63.6) (width 0.7) (layer F.Cu) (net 9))
 (segment (start 144.45 63.6) (end 145.15 62.9) (width 0.7) (layer F.Cu) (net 9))
 (segment (start 108.05 63.1) (end 109.9 63.1) (width 0.7) (layer F.Cu) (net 10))
 (segment (start 109.9 63.1) (end 110.6 63.8) (width 0.7) (layer F.Cu) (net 10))
 (segment (start 118.15 92.8) (end 117.7 92.8) (width 0.7) (layer F.Cu) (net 42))
 (segment (start 117.7 92.8) (end 117.415 92.515) (width 0.7) (layer F.Cu) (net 42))
 (segment (start 117.415 92.515) (end 117.415 91.565) (width 0.7) (layer F.Cu) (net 42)))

